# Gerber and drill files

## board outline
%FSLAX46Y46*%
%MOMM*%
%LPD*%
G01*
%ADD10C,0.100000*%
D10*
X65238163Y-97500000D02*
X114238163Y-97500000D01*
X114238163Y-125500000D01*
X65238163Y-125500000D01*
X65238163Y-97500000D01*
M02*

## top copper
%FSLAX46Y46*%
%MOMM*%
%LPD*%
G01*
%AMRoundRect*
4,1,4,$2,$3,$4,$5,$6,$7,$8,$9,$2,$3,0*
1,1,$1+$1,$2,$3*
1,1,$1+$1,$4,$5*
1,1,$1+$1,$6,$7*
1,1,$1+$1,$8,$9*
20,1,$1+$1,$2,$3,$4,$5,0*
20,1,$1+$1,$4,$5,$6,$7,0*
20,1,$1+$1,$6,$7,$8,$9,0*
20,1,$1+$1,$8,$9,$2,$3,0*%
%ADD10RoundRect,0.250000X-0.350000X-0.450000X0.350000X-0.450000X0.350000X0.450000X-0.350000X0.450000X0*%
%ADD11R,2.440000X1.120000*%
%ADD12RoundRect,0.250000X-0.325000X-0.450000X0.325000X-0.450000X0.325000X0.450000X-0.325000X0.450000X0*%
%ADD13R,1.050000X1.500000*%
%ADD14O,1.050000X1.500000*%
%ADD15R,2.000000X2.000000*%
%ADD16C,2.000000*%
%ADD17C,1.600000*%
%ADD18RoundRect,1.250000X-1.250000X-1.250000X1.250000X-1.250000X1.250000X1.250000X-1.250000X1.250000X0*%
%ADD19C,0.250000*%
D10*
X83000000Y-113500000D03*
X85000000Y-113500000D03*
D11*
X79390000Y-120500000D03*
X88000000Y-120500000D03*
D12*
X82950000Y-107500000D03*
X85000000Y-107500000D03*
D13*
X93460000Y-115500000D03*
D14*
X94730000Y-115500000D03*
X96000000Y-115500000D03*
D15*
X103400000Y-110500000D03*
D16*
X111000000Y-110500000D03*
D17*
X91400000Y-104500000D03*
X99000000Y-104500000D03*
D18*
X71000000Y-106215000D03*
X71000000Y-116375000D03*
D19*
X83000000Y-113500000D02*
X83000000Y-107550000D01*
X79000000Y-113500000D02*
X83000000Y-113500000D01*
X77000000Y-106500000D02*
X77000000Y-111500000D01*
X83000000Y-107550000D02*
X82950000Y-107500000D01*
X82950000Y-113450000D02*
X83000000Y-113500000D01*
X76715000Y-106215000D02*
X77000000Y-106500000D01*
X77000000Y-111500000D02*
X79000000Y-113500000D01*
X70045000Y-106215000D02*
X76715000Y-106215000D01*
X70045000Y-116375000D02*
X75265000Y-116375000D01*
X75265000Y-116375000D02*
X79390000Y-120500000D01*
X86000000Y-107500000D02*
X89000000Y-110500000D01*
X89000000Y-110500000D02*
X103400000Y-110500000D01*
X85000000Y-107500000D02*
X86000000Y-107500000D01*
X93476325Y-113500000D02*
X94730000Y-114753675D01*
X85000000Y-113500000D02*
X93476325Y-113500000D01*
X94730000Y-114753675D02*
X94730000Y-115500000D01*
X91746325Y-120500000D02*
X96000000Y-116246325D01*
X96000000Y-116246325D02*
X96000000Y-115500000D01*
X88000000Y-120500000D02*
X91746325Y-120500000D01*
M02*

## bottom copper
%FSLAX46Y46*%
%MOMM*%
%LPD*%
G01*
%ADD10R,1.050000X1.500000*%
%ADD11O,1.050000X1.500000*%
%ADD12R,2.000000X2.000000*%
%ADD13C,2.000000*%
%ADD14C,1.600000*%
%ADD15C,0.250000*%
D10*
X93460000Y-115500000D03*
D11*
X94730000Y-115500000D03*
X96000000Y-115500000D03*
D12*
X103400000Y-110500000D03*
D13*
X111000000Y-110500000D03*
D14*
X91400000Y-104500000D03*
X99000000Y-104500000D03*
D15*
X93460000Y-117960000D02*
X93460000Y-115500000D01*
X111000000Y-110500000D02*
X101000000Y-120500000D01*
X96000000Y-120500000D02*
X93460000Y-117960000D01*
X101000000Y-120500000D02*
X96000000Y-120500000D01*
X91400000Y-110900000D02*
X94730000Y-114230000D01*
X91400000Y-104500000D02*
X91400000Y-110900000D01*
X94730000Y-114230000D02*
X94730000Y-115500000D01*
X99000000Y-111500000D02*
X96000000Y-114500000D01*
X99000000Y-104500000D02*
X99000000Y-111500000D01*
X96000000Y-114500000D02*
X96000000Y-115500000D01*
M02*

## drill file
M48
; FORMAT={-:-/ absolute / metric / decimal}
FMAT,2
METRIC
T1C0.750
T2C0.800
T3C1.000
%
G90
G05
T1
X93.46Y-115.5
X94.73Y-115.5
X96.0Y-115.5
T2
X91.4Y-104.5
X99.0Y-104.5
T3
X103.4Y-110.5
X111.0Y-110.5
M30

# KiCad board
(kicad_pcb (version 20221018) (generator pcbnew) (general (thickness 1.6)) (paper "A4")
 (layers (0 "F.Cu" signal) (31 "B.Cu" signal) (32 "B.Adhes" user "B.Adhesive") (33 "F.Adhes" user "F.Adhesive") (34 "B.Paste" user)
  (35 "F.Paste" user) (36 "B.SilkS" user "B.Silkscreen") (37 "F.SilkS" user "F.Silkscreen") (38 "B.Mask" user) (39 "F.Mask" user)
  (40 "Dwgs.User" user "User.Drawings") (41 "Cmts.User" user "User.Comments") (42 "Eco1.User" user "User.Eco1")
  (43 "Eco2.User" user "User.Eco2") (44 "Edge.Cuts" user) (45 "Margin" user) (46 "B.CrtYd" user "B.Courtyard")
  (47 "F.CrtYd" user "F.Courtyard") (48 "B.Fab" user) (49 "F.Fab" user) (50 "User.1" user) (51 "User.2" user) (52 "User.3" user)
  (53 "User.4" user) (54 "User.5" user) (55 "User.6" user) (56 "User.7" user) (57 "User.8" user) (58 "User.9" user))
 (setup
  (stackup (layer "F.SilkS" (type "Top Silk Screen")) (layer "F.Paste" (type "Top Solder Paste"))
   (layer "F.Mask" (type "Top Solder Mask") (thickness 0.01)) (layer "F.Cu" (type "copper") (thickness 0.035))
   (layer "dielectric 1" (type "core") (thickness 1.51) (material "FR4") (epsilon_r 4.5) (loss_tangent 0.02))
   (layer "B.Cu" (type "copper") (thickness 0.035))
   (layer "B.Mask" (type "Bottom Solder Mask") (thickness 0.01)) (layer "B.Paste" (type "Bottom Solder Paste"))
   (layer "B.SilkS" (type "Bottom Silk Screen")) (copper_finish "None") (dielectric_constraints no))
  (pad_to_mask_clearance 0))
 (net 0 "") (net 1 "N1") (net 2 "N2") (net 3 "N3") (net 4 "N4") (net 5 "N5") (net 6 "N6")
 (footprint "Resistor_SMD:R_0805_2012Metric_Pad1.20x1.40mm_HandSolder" (layer "F.Cu") (at 84 113.5)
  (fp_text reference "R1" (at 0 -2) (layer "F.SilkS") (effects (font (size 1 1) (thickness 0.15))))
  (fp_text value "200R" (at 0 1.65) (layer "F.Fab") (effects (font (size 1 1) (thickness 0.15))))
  (pad "1" smd roundrect (at -1 0) (size 1.2 1.4) (layers "F.Cu" "F.Paste" "F.Mask") (roundrect_rratio 0.208333) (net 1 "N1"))
  (pad "2" smd roundrect (at 1 0) (size 1.2 1.4) (layers "F.Cu" "F.Paste" "F.Mask") (roundrect_rratio 0.208333) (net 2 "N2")))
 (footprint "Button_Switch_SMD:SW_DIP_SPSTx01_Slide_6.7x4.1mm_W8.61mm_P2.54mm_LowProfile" (layer "F.Cu") (at 83.695 120.5)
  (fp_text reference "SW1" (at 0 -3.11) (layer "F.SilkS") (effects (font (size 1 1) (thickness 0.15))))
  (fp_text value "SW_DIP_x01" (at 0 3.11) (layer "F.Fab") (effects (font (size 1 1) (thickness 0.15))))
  (pad "1" smd rect (at -4.305 0) (size 2.44 1.12) (layers "F.Cu" "F.Paste" "F.Mask") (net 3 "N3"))
  (pad "2" smd rect (at 4.305 0) (size 2.44 1.12) (layers "F.Cu" "F.Paste" "F.Mask") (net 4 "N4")))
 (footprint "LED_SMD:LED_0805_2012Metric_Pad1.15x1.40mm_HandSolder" (layer "F.Cu") (at 83.975 107.5)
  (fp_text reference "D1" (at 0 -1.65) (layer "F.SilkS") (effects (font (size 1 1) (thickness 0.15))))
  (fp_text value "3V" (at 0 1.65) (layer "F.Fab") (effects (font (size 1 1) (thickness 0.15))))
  (pad "1" smd roundrect (at -1.025 0) (size 1.15 1.4) (layers "F.Cu" "F.Paste" "F.Mask") (roundrect_rratio 0.217391) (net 1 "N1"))
  (pad "2" smd roundrect (at 1.025 0) (size 1.15 1.4) (layers "F.Cu" "F.Paste" "F.Mask") (roundrect_rratio 0.217391) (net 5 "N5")))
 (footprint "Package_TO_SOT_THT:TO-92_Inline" (layer "F.Cu") (at 93.46 115.5)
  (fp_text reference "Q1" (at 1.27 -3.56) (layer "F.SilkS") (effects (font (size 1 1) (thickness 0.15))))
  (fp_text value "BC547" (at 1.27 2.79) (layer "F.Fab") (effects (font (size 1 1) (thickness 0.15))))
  (pad "1" thru_hole rect (at 0 0) (size 1.05 1.5) (drill 0.75) (layers "*.Cu" "*.Mask") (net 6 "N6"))
  (pad "2" thru_hole oval (at 1.27 0) (size 1.05 1.5) (drill 0.75) (layers "*.Cu" "*.Mask") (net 2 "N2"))
  (pad "3" thru_hole oval (at 2.54 0) (size 1.05 1.5) (drill 0.75) (layers "*.Cu" "*.Mask") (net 4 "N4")))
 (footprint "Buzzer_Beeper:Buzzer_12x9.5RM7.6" (layer "F.Cu") (at 103.4 110.5)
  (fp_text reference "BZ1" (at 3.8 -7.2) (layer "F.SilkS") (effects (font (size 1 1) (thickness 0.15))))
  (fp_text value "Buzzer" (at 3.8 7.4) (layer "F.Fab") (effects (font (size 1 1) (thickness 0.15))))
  (pad "1" thru_hole rect (at 0 0) (size 2 2) (drill 1) (layers "*.Cu" "*.Mask") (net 5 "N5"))
  (pad "2" thru_hole circle (at 7.6 0) (size 2 2) (drill 1) (layers "*.Cu" "*.Mask") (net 6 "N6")))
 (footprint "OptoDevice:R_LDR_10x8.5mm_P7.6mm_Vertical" (layer "F.Cu") (at 91.4 104.5)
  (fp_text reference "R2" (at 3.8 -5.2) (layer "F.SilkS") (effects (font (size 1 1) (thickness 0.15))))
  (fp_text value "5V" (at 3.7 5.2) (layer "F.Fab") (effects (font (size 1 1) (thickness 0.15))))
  (pad "1" thru_hole circle (at 0 0) (size 1.6 1.6) (drill 0.8) (layers "*.Cu" "*.Mask") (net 2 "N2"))
  (pad "2" thru_hole circle (at 7.6 0) (size 1.6 1.6) (drill 0.8) (layers "*.Cu" "*.Mask") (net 4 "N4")))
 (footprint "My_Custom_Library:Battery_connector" (layer "F.Cu") (at 71 111.295)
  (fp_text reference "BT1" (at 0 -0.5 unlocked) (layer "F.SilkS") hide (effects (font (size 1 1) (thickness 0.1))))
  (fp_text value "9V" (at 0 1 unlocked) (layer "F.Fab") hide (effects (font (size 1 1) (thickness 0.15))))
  (pad "1" smd roundrect (at 0 -5.08) (size 5 5) (layers "F.Cu" "F.Paste" "F.Mask") (roundrect_rratio 0.25) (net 1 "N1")
   (thermal_bridge_angle 45))
  (pad "2" smd roundrect (at 0 5.08) (size 5 5) (layers "F.Cu" "F.Paste" "F.Mask") (roundrect_rratio 0.25) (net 3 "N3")
   (thermal_bridge_angle 45)))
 (gr_rect (start 65.238163 97.5) (end 114.238163 125.5) (stroke (width 0.1) (type default)) (fill none) (layer "Edge.Cuts"))
 (segment (start 83 113.5) (end 83 107.55) (width 0.25) (layer "F.Cu") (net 1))
 (segment (start 79 113.5) (end 83 113.5) (width 0.25) (layer "F.Cu") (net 1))
 (segment (start 77 106.5) (end 77 111.5) (width 0.25) (layer "F.Cu") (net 1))
 (segment (start 83 107.55) (end 82.95 107.5) (width 0.25) (layer "F.Cu") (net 1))
 (segment (start 82.95 113.45) (end 83 113.5) (width 0.25) (layer "F.Cu") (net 1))
 (segment (start 76.715 106.215) (end 77 106.5) (width 0.25) (layer "F.Cu") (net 1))
 (segment (start 77 111.5) (end 79 113.5) (width 0.25) (layer "F.Cu") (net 1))
 (segment (start 70.045 106.215) (end 76.715 106.215) (width 0.25) (layer "F.Cu") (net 1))
 (segment (start 70.045 116.375) (end 75.265 116.375) (width 0.25) (layer "F.Cu") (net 3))
 (segment (start 75.265 116.375) (end 79.39 120.5) (width 0.25) (layer "F.Cu") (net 3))
 (segment (start 86 107.5) (end 89 110.5) (width 0.25) (layer "F.Cu") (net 5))
 (segment (start 89 110.5) (end 103.4 110.5) (width 0.25) (layer "F.Cu") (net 5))
 (segment (start 85 107.5) (end 86 107.5) (width 0.25) (layer "F.Cu") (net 5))
 (segment (start 93.46 117.96) (end 93.46 115.5) (width 0.25) (layer "B.Cu") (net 6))
 (segment (start 111 110.5) (end 101 120.5) (width 0.25) (layer "B.Cu") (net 6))
 (segment (start 96 120.5) (end 93.46 117.96) (width 0.25) (layer "B.Cu") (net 6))
 (segment (start 101 120.5) (end 96 120.5) (width 0.25) (layer "B.Cu") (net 6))
 (segment (start 93.476325 113.5) (end 94.73 114.753675) (width 0.25) (layer "F.Cu") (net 2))
 (segment (start 85 113.5) (end 93.476325 113.5) (width 0.25) (layer "F.Cu") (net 2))
 (segment (start 94.73 114.753675) (end 94.73 115.5) (width 0.25) (layer "F.Cu") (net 2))
 (segment (start 91.4 110.9) (end 94.73 114.23) (width 0.25) (layer "B.Cu") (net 2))
 (segment (start 91.4 104.5) (end 91.4 110.9) (width 0.25) (layer "B.Cu") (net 2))
 (segment (start 94.73 114.23) (end 94.73 115.5) (width 0.25) (layer "B.Cu") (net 2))
 (segment (start 91.746325 120.5) (end 96 116.246325) (width 0.25) (layer "F.Cu") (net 4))
 (segment (start 96 116.246325) (end 96 115.5) (width 0.25) (layer "F.Cu") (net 4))
 (segment (start 88 120.5) (end 91.746325 120.5) (width 0.25) (layer "F.Cu") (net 4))
 (segment (start 99 111.5) (end 96 114.5) (width 0.25) (layer "B.Cu") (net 4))
 (segment (start 99 104.5) (end 99 111.5) (width 0.25) (layer "B.Cu") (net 4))
 (segment (start 96 114.5) (end 96 115.5) (width 0.25) (layer "B.Cu") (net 4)))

